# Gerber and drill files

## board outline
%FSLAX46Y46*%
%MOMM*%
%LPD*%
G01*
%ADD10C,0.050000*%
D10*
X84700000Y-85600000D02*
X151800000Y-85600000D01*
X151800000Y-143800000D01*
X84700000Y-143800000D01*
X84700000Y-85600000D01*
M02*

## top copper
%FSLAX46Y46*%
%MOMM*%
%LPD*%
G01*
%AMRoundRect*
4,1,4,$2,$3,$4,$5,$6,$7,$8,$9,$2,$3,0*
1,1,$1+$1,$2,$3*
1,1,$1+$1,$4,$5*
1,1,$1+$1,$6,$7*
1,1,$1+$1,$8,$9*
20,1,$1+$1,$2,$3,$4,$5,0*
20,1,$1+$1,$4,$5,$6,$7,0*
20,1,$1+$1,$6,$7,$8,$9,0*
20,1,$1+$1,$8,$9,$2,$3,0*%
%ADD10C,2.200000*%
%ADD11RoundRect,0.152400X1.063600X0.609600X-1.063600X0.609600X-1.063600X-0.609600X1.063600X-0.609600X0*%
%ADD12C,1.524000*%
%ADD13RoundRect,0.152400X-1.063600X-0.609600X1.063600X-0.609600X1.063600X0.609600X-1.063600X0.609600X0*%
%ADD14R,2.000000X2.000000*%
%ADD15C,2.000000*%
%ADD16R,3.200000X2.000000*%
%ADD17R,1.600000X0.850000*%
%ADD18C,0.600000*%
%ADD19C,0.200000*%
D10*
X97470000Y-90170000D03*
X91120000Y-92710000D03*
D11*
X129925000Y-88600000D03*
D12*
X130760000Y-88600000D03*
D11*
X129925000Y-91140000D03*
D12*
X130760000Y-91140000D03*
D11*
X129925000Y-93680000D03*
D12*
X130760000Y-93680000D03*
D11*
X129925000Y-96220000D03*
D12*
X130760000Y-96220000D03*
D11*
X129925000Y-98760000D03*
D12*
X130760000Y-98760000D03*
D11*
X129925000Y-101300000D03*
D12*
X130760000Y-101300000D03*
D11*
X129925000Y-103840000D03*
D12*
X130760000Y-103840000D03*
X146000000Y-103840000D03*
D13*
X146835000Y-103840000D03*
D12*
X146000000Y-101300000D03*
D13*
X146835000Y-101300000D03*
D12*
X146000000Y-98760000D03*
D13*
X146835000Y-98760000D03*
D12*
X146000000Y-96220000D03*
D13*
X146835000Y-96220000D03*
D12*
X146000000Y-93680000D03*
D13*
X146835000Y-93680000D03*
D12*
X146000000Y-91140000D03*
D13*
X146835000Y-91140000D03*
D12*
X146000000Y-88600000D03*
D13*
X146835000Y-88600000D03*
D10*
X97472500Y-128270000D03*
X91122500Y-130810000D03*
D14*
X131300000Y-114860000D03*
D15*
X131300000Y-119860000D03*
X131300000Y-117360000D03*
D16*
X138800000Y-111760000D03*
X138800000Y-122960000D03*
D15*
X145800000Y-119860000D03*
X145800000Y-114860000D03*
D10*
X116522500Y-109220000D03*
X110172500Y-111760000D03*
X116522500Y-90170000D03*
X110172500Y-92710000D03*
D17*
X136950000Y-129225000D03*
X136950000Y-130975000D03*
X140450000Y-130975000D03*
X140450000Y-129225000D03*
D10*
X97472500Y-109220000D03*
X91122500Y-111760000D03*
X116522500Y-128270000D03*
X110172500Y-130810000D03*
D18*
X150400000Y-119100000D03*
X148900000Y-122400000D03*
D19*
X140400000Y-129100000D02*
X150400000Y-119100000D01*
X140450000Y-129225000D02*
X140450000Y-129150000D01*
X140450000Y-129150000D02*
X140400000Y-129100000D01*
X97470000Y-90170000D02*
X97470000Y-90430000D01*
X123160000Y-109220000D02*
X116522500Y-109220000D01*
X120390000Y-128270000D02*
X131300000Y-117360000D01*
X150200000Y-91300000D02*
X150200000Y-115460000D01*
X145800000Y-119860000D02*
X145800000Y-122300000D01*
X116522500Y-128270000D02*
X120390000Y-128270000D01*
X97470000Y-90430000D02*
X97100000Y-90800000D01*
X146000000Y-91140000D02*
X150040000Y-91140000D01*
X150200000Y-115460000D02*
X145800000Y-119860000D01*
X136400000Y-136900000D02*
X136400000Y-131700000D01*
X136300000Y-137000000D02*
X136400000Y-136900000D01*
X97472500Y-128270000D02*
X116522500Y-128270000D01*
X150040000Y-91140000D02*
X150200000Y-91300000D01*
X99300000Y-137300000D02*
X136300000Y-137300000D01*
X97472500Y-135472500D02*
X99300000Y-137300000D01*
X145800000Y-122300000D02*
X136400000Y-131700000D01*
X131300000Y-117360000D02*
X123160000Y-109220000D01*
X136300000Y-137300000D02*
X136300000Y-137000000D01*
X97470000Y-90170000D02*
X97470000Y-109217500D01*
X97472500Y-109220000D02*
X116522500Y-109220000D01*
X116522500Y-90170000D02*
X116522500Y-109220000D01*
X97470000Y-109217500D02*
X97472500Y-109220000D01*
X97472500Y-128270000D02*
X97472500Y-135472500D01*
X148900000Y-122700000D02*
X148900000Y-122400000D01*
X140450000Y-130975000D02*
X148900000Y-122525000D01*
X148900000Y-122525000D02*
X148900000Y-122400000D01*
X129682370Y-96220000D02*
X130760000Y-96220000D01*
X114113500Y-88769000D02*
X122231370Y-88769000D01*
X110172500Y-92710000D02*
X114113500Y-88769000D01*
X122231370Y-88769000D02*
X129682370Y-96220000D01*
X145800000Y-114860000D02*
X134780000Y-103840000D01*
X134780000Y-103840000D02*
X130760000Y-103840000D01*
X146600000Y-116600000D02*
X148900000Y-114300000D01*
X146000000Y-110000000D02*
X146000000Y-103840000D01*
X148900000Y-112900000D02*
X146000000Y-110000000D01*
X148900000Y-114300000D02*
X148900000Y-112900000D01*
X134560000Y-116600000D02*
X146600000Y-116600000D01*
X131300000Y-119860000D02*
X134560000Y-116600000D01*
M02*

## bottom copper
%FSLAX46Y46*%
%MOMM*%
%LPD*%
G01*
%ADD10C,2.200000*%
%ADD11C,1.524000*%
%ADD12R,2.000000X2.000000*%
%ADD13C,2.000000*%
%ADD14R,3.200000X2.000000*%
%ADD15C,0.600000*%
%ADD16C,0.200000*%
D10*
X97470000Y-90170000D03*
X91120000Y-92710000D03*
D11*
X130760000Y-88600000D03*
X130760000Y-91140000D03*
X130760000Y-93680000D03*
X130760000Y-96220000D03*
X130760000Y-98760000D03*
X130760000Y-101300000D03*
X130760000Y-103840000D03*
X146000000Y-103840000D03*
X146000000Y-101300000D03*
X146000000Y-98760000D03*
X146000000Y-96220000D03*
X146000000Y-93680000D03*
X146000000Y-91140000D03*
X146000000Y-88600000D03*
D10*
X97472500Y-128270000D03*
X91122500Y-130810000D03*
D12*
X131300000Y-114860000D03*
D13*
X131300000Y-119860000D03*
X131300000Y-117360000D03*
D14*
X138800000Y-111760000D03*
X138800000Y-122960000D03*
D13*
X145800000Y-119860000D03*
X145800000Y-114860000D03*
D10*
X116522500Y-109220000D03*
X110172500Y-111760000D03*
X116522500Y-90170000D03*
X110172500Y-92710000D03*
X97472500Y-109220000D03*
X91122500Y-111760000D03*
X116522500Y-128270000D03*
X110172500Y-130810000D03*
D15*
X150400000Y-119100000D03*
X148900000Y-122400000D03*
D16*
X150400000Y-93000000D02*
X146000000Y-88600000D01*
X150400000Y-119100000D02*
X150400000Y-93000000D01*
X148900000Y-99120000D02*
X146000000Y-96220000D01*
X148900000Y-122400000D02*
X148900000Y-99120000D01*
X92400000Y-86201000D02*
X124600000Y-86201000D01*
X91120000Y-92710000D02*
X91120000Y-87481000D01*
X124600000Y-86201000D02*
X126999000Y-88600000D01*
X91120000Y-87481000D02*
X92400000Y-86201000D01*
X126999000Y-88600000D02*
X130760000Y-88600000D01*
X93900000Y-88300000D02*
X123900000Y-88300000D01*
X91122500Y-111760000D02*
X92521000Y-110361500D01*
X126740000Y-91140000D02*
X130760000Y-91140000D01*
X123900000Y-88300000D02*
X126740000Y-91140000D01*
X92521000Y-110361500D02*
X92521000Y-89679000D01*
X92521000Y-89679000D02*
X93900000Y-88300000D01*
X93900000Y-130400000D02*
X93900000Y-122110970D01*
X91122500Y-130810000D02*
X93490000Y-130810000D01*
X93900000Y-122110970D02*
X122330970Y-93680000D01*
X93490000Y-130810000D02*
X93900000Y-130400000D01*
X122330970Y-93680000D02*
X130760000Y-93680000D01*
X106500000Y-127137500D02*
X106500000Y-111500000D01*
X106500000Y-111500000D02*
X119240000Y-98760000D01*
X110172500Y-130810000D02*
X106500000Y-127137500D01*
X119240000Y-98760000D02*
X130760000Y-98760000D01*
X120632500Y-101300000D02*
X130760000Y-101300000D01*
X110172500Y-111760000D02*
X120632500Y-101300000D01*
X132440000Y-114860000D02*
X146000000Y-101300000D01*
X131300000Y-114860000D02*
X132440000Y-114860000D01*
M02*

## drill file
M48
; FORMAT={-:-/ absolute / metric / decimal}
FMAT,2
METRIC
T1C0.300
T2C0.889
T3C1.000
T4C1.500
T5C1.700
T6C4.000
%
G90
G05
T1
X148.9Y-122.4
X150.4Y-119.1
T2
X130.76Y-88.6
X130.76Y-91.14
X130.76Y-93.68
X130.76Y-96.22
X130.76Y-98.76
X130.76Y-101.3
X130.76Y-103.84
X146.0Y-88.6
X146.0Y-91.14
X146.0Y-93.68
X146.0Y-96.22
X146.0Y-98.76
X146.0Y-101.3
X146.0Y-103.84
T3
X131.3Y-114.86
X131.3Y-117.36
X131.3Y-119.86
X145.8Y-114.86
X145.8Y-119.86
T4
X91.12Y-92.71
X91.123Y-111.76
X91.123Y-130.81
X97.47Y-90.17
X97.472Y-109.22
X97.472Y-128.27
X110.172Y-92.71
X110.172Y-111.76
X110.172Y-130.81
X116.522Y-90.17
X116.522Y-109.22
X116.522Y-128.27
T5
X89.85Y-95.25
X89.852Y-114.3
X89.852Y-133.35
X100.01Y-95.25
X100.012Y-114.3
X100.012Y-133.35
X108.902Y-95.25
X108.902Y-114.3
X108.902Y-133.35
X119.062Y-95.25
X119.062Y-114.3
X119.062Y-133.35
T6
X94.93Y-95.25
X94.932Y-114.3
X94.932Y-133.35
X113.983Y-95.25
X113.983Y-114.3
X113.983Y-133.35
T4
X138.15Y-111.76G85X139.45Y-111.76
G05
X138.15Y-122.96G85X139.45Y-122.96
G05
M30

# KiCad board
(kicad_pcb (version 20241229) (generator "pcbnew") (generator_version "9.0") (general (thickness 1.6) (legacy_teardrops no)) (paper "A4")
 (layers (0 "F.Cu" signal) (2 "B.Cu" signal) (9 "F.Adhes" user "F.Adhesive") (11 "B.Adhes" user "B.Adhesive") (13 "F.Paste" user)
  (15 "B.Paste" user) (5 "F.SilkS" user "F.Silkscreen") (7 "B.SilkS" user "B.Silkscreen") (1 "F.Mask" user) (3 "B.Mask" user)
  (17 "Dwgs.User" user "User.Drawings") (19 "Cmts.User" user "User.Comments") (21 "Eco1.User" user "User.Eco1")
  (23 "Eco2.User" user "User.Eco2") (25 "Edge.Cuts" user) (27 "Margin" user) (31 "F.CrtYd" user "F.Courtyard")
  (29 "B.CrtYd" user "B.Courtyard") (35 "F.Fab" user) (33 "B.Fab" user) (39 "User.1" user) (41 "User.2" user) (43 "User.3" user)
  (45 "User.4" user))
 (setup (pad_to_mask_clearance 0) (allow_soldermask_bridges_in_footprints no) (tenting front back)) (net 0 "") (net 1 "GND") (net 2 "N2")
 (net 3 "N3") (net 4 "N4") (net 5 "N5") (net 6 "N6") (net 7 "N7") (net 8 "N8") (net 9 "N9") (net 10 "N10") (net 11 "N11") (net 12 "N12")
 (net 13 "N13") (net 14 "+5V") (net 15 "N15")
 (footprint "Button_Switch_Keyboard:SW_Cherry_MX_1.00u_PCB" (layer "F.Cu") (at 97.47 90.17)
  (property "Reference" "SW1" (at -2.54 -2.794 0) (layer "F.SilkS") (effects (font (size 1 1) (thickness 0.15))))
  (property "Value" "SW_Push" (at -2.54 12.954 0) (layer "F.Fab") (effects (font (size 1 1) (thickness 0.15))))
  (pad "" np_thru_hole circle (at -7.62 5.08) (size 1.7 1.7) (drill 1.7) (layers "*.Cu" "*.Mask"))
  (pad "" np_thru_hole circle (at -2.54 5.08) (size 4 4) (drill 4) (layers "*.Cu" "*.Mask"))
  (pad "" np_thru_hole circle (at 2.54 5.08) (size 1.7 1.7) (drill 1.7) (layers "*.Cu" "*.Mask"))
  (pad "1" thru_hole circle (at 0 0) (size 2.2 2.2) (drill 1.5) (layers "*.Cu" "*.Mask") (remove_unused_layers no) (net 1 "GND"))
  (pad "2" thru_hole circle (at -6.35 2.54) (size 2.2 2.2) (drill 1.5) (layers "*.Cu" "*.Mask") (remove_unused_layers no) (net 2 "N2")))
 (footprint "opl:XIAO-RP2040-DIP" (layer "F.Cu") (at 138.38 96.22)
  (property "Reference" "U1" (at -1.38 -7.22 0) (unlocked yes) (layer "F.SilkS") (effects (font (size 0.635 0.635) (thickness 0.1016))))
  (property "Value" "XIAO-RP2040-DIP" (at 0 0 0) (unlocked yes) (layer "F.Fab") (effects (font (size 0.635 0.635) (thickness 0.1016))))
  (pad "1" smd roundrect (at -8.455 -7.62 180) (size 2.432 1.524) (layers "F.Cu" "F.Mask") (roundrect_rratio 0.1) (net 2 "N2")
   (thermal_bridge_angle 45))
  (pad "1" thru_hole circle (at -7.62 -7.62 180) (size 1.524 1.524) (drill 0.889) (layers "*.Cu" "*.Mask") (remove_unused_layers no)
   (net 2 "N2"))
  (pad "2" smd roundrect (at -8.455 -5.08 180) (size 2.432 1.524) (layers "F.Cu" "F.Mask") (roundrect_rratio 0.1) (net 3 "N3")
   (thermal_bridge_angle 45))
  (pad "2" thru_hole circle (at -7.62 -5.08 180) (size 1.524 1.524) (drill 0.889) (layers "*.Cu" "*.Mask") (remove_unused_layers no)
   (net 3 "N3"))
  (pad "3" smd roundrect (at -8.455 -2.54 180) (size 2.432 1.524) (layers "F.Cu" "F.Mask") (roundrect_rratio 0.1) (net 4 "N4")
   (thermal_bridge_angle 45))
  (pad "3" thru_hole circle (at -7.62 -2.54 180) (size 1.524 1.524) (drill 0.889) (layers "*.Cu" "*.Mask") (remove_unused_layers no)
   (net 4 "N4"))
  (pad "4" smd roundrect (at -8.455 0 180) (size 2.432 1.524) (layers "F.Cu" "F.Mask") (roundrect_rratio 0.1) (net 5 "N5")
   (thermal_bridge_angle 45))
  (pad "4" thru_hole circle (at -7.62 0 180) (size 1.524 1.524) (drill 0.889) (layers "*.Cu" "*.Mask") (remove_unused_layers no)
   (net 5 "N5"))
  (pad "5" smd roundrect (at -8.455 2.54 180) (size 2.432 1.524) (layers "F.Cu" "F.Mask") (roundrect_rratio 0.1) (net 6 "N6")
   (thermal_bridge_angle 45))
  (pad "5" thru_hole circle (at -7.62 2.54 180) (size 1.524 1.524) (drill 0.889) (layers "*.Cu" "*.Mask") (remove_unused_layers no)
   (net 6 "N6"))
  (pad "6" smd roundrect (at -8.455 5.08 180) (size 2.432 1.524) (layers "F.Cu" "F.Mask") (roundrect_rratio 0.1) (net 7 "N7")
   (thermal_bridge_angle 45))
  (pad "6" thru_hole circle (at -7.62 5.08 180) (size 1.524 1.524) (drill 0.889) (layers "*.Cu" "*.Mask") (remove_unused_layers no)
   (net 7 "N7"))
  (pad "7" smd roundrect (at -8.455 7.62 180) (size 2.432 1.524) (layers "F.Cu" "F.Mask") (roundrect_rratio 0.1) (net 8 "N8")
   (thermal_bridge_angle 45))
  (pad "7" thru_hole circle (at -7.62 7.62 180) (size 1.524 1.524) (drill 0.889) (layers "*.Cu" "*.Mask") (remove_unused_layers no)
   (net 8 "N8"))
  (pad "8" thru_hole circle (at 7.62 7.62) (size 1.524 1.524) (drill 0.889) (layers "*.Cu" "*.Mask") (remove_unused_layers no) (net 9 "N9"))
  (pad "8" smd roundrect (at 8.455 7.62) (size 2.432 1.524) (layers "F.Cu" "F.Mask") (roundrect_rratio 0.1) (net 9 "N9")
   (thermal_bridge_angle 45))
  (pad "9" thru_hole circle (at 7.62 5.08) (size 1.524 1.524) (drill 0.889) (layers "*.Cu" "*.Mask") (remove_unused_layers no)
   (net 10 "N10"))
  (pad "9" smd roundrect (at 8.455 5.08) (size 2.432 1.524) (layers "F.Cu" "F.Mask") (roundrect_rratio 0.1) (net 10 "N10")
   (thermal_bridge_angle 45))
  (pad "10" thru_hole circle (at 7.62 2.54) (size 1.524 1.524) (drill 0.889) (layers "*.Cu" "*.Mask") (remove_unused_layers no)
   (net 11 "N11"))
  (pad "10" smd roundrect (at 8.455 2.54) (size 2.432 1.524) (layers "F.Cu" "F.Mask") (roundrect_rratio 0.1) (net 11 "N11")
   (thermal_bridge_angle 45))
  (pad "11" thru_hole circle (at 7.62 0) (size 1.524 1.524) (drill 0.889) (layers "*.Cu" "*.Mask") (remove_unused_layers no) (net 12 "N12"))
  (pad "11" smd roundrect (at 8.455 0) (size 2.432 1.524) (layers "F.Cu" "F.Mask") (roundrect_rratio 0.1) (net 12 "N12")
   (thermal_bridge_angle 45))
  (pad "12" thru_hole circle (at 7.62 -2.54) (size 1.524 1.524) (drill 0.889) (layers "*.Cu" "*.Mask") (remove_unused_layers no)
   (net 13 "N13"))
  (pad "12" smd roundrect (at 8.455 -2.54) (size 2.432 1.524) (layers "F.Cu" "F.Mask") (roundrect_rratio 0.1) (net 13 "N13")
   (thermal_bridge_angle 45))
  (pad "13" thru_hole circle (at 7.62 -5.08) (size 1.524 1.524) (drill 0.889) (layers "*.Cu" "*.Mask") (remove_unused_layers no)
   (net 1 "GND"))
  (pad "13" smd roundrect (at 8.455 -5.08) (size 2.432 1.524) (layers "F.Cu" "F.Mask") (roundrect_rratio 0.1) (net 1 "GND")
   (thermal_bridge_angle 45))
  (pad "14" thru_hole circle (at 7.62 -7.62) (size 1.524 1.524) (drill 0.889) (layers "*.Cu" "*.Mask") (remove_unused_layers no)
   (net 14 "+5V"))
  (pad "14" smd roundrect (at 8.455 -7.62) (size 2.432 1.524) (layers "F.Cu" "F.Mask") (roundrect_rratio 0.1) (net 14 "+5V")
   (thermal_bridge_angle 45)))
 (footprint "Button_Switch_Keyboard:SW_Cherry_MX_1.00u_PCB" (layer "F.Cu") (at 97.4725 128.27)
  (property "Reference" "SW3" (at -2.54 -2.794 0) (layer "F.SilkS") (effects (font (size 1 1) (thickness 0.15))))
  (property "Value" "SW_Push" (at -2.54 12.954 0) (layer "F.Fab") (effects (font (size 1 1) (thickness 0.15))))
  (pad "" np_thru_hole circle (at -7.62 5.08) (size 1.7 1.7) (drill 1.7) (layers "*.Cu" "*.Mask"))
  (pad "" np_thru_hole circle (at -2.54 5.08) (size 4 4) (drill 4) (layers "*.Cu" "*.Mask"))
  (pad "" np_thru_hole circle (at 2.54 5.08) (size 1.7 1.7) (drill 1.7) (layers "*.Cu" "*.Mask"))
  (pad "1" thru_hole circle (at 0 0) (size 2.2 2.2) (drill 1.5) (layers "*.Cu" "*.Mask") (remove_unused_layers no) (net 1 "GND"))
  (pad "2" thru_hole circle (at -6.35 2.54) (size 2.2 2.2) (drill 1.5) (layers "*.Cu" "*.Mask") (remove_unused_layers no) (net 4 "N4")))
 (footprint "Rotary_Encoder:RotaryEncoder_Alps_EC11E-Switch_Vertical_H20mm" (layer "F.Cu") (at 131.3 114.86)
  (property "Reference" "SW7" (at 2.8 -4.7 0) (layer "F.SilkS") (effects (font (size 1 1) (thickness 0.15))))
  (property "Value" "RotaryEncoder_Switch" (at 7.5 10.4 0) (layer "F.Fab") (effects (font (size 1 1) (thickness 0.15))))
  (pad "A" thru_hole rect (at 0 0) (size 2 2) (drill 1) (layers "*.Cu" "*.Mask") (remove_unused_layers no) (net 10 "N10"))
  (pad "B" thru_hole circle (at 0 5) (size 2 2) (drill 1) (layers "*.Cu" "*.Mask") (remove_unused_layers no) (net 9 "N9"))
  (pad "C" thru_hole circle (at 0 2.5) (size 2 2) (drill 1) (layers "*.Cu" "*.Mask") (remove_unused_layers no) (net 1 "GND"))
  (pad "MP" thru_hole rect (at 7.5 -3.1) (size 3.2 2) (drill oval 2.8 1.5) (layers "*.Cu" "*.Mask") (remove_unused_layers no))
  (pad "MP" thru_hole rect (at 7.5 8.1) (size 3.2 2) (drill oval 2.8 1.5) (layers "*.Cu" "*.Mask") (remove_unused_layers no))
  (pad "S1" thru_hole circle (at 14.5 5) (size 2 2) (drill 1) (layers "*.Cu" "*.Mask") (remove_unused_layers no) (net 1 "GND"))
  (pad "S2" thru_hole circle (at 14.5 0) (size 2 2) (drill 1) (layers "*.Cu" "*.Mask") (remove_unused_layers no) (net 8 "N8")))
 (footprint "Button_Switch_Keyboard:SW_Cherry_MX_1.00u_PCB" (layer "F.Cu") (at 116.5225 109.22)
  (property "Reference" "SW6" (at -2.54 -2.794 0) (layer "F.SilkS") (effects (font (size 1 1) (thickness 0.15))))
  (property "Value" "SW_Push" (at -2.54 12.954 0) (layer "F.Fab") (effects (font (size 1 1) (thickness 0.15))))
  (pad "" np_thru_hole circle (at -7.62 5.08) (size 1.7 1.7) (drill 1.7) (layers "*.Cu" "*.Mask"))
  (pad "" np_thru_hole circle (at -2.54 5.08) (size 4 4) (drill 4) (layers "*.Cu" "*.Mask"))
  (pad "" np_thru_hole circle (at 2.54 5.08) (size 1.7 1.7) (drill 1.7) (layers "*.Cu" "*.Mask"))
  (pad "1" thru_hole circle (at 0 0) (size 2.2 2.2) (drill 1.5) (layers "*.Cu" "*.Mask") (remove_unused_layers no) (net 1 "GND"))
  (pad "2" thru_hole circle (at -6.35 2.54) (size 2.2 2.2) (drill 1.5) (layers "*.Cu" "*.Mask") (remove_unused_layers no) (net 7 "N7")))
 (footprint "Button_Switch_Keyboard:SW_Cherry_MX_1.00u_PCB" (layer "F.Cu") (at 116.5225 90.17)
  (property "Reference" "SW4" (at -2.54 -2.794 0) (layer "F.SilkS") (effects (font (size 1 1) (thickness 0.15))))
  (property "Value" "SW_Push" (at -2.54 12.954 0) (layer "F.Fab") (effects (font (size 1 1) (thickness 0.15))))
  (pad "" np_thru_hole circle (at -7.62 5.08) (size 1.7 1.7) (drill 1.7) (layers "*.Cu" "*.Mask"))
  (pad "" np_thru_hole circle (at -2.54 5.08) (size 4 4) (drill 4) (layers "*.Cu" "*.Mask"))
  (pad "" np_thru_hole circle (at 2.54 5.08) (size 1.7 1.7) (drill 1.7) (layers "*.Cu" "*.Mask"))
  (pad "1" thru_hole circle (at 0 0) (size 2.2 2.2) (drill 1.5) (layers "*.Cu" "*.Mask") (remove_unused_layers no) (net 1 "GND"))
  (pad "2" thru_hole circle (at -6.35 2.54) (size 2.2 2.2) (drill 1.5) (layers "*.Cu" "*.Mask") (remove_unused_layers no) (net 5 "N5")))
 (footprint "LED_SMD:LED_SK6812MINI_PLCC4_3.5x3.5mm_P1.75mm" (layer "F.Cu") (at 138.7 130.1)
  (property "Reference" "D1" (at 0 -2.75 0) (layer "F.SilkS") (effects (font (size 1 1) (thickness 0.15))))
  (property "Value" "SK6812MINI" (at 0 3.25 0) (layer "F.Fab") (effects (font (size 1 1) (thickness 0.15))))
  (pad "1" smd rect (at -1.75 -0.875) (size 1.6 0.85) (layers "F.Cu" "F.Mask" "F.Paste") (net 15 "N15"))
  (pad "2" smd rect (at -1.75 0.875) (size 1.6 0.85) (layers "F.Cu" "F.Mask" "F.Paste") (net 1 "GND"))
  (pad "3" smd rect (at 1.75 0.875) (size 1.6 0.85) (layers "F.Cu" "F.Mask" "F.Paste") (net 12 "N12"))
  (pad "4" smd rect (at 1.75 -0.875) (size 1.6 0.85) (layers "F.Cu" "F.Mask" "F.Paste") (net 14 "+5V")))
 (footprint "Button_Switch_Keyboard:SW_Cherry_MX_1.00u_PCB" (layer "F.Cu") (at 97.4725 109.22)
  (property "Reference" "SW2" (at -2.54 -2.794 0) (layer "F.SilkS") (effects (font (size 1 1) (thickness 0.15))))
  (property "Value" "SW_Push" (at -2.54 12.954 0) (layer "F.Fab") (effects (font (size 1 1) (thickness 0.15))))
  (pad "" np_thru_hole circle (at -7.62 5.08) (size 1.7 1.7) (drill 1.7) (layers "*.Cu" "*.Mask"))
  (pad "" np_thru_hole circle (at -2.54 5.08) (size 4 4) (drill 4) (layers "*.Cu" "*.Mask"))
  (pad "" np_thru_hole circle (at 2.54 5.08) (size 1.7 1.7) (drill 1.7) (layers "*.Cu" "*.Mask"))
  (pad "1" thru_hole circle (at 0 0) (size 2.2 2.2) (drill 1.5) (layers "*.Cu" "*.Mask") (remove_unused_layers no) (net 1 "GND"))
  (pad "2" thru_hole circle (at -6.35 2.54) (size 2.2 2.2) (drill 1.5) (layers "*.Cu" "*.Mask") (remove_unused_layers no) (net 3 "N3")))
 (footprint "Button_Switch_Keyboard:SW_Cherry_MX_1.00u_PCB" (layer "F.Cu") (at 116.5225 128.27)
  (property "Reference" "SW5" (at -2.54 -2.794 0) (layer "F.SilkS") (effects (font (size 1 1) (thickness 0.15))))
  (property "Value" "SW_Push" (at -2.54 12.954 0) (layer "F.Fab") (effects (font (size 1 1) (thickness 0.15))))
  (pad "" np_thru_hole circle (at -7.62 5.08) (size 1.7 1.7) (drill 1.7) (layers "*.Cu" "*.Mask"))
  (pad "" np_thru_hole circle (at -2.54 5.08) (size 4 4) (drill 4) (layers "*.Cu" "*.Mask"))
  (pad "" np_thru_hole circle (at 2.54 5.08) (size 1.7 1.7) (drill 1.7) (layers "*.Cu" "*.Mask"))
  (pad "1" thru_hole circle (at 0 0) (size 2.2 2.2) (drill 1.5) (layers "*.Cu" "*.Mask") (remove_unused_layers no) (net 1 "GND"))
  (pad "2" thru_hole circle (at -6.35 2.54) (size 2.2 2.2) (drill 1.5) (layers "*.Cu" "*.Mask") (remove_unused_layers no) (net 6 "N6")))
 (gr_rect (start 84.7 85.6) (end 151.8 143.8) (stroke (width 0.05) (type default)) (fill no) (layer "Edge.Cuts"))
 (segment (start 140.4 129.1) (end 150.4 119.1) (width 0.2) (layer "F.Cu") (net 14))
 (segment (start 140.45 129.225) (end 140.45 129.15) (width 0.2) (layer "F.Cu") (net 14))
 (segment (start 140.45 129.15) (end 140.4 129.1) (width 0.2) (layer "F.Cu") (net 14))
 (via (at 150.4 119.1) (size 0.6) (drill 0.3) (layers "F.Cu" "B.Cu") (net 14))
 (segment (start 150.4 93) (end 146 88.6) (width 0.2) (layer "B.Cu") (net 14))
 (segment (start 150.4 119.1) (end 150.4 93) (width 0.2) (layer "B.Cu") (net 14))
 (segment (start 97.47 90.17) (end 97.47 90.43) (width 0.2) (layer "F.Cu") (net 1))
 (segment (start 123.16 109.22) (end 116.5225 109.22) (width 0.2) (layer "F.Cu") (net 1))
 (segment (start 120.39 128.27) (end 131.3 117.36) (width 0.2) (layer "F.Cu") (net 1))
 (segment (start 150.2 91.3) (end 150.2 115.46) (width 0.2) (layer "F.Cu") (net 1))
 (segment (start 145.8 119.86) (end 145.8 122.3) (width 0.2) (layer "F.Cu") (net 1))
 (segment (start 116.5225 128.27) (end 120.39 128.27) (width 0.2) (layer "F.Cu") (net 1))
 (segment (start 97.47 90.43) (end 97.1 90.8) (width 0.2) (layer "F.Cu") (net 1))
 (segment (start 146 91.14) (end 150.04 91.14) (width 0.2) (layer "F.Cu") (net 1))
 (segment (start 150.2 115.46) (end 145.8 119.86) (width 0.2) (layer "F.Cu") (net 1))
 (segment (start 136.4 136.9) (end 136.4 131.7) (width 0.2) (layer "F.Cu") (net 1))
 (segment (start 136.3 137) (end 136.4 136.9) (width 0.2) (layer "F.Cu") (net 1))
 (segment (start 97.4725 128.27) (end 116.5225 128.27) (width 0.2) (layer "F.Cu") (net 1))
 (segment (start 150.04 91.14) (end 150.2 91.3) (width 0.2) (layer "F.Cu") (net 1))
 (segment (start 99.3 137.3) (end 136.3 137.3) (width 0.2) (layer "F.Cu") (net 1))
 (segment (start 97.4725 135.4725) (end 99.3 137.3) (width 0.2) (layer "F.Cu") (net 1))
 (segment (start 145.8 122.3) (end 136.4 131.7) (width 0.2) (layer "F.Cu") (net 1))
 (segment (start 131.3 117.36) (end 123.16 109.22) (width 0.2) (layer "F.Cu") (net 1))
 (segment (start 136.3 137.3) (end 136.3 137) (width 0.2) (layer "F.Cu") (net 1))
 (segment (start 97.47 90.17) (end 97.47 109.2175) (width 0.2) (layer "F.Cu") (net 1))
 (segment (start 97.4725 109.22) (end 116.5225 109.22) (width 0.2) (layer "F.Cu") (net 1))
 (segment (start 116.5225 90.17) (end 116.5225 109.22) (width 0.2) (layer "F.Cu") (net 1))
 (segment (start 97.47 109.2175) (end 97.4725 109.22) (width 0.2) (layer "F.Cu") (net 1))
 (segment (start 97.4725 128.27) (end 97.4725 135.4725) (width 0.2) (layer "F.Cu") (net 1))
 (segment (start 148.9 122.7) (end 148.9 122.4) (width 0.2) (layer "F.Cu") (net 12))
 (segment (start 140.45 130.975) (end 148.9 122.525) (width 0.2) (layer "F.Cu") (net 12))
 (segment (start 148.9 122.525) (end 148.9 122.4) (width 0.2) (layer "F.Cu") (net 12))
 (via (at 148.9 122.4) (size 0.6) (drill 0.3) (layers "F.Cu" "B.Cu") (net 12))
 (segment (start 148.9 99.12) (end 146 96.22) (width 0.2) (layer "B.Cu") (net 12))
 (segment (start 148.9 122.4) (end 148.9 99.12) (width 0.2) (layer "B.Cu") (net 12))
 (segment (start 92.4 86.201) (end 124.6 86.201) (width 0.2) (layer "B.Cu") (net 2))
 (segment (start 91.12 92.71) (end 91.12 87.481) (width 0.2) (layer "B.Cu") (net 2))
 (segment (start 124.6 86.201) (end 126.999 88.6) (width 0.2) (layer "B.Cu") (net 2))
 (segment (start 91.12 87.481) (end 92.4 86.201) (width 0.2) (layer "B.Cu") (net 2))
 (segment (start 126.999 88.6) (end 130.76 88.6) (width 0.2) (layer "B.Cu") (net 2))
 (segment (start 93.9 88.3) (end 123.9 88.3) (width 0.2) (layer "B.Cu") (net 3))
 (segment (start 91.1225 111.76) (end 92.521 110.3615) (width 0.2) (layer "B.Cu") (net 3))
 (segment (start 126.74 91.14) (end 130.76 91.14) (width 0.2) (layer "B.Cu") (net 3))
 (segment (start 123.9 88.3) (end 126.74 91.14) (width 0.2) (layer "B.Cu") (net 3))
 (segment (start 92.521 110.3615) (end 92.521 89.679) (width 0.2) (layer "B.Cu") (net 3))
 (segment (start 92.521 89.679) (end 93.9 88.3) (width 0.2) (layer "B.Cu") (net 3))
 (segment (start 93.9 130.4) (end 93.9 122.11097) (width 0.2) (layer "B.Cu") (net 4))
 (segment (start 91.1225 130.81) (end 93.49 130.81) (width 0.2) (layer "B.Cu") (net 4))
 (segment (start 93.9 122.11097) (end 122.33097 93.68) (width 0.2) (layer "B.Cu") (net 4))
 (segment (start 93.49 130.81) (end 93.9 130.4) (width 0.2) (layer "B.Cu") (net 4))
 (segment (start 122.33097 93.68) (end 130.76 93.68) (width 0.2) (layer "B.Cu") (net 4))
 (segment (start 129.68237 96.22) (end 130.76 96.22) (width 0.2) (layer "F.Cu") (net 5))
 (segment (start 114.1135 88.769) (end 122.23137 88.769) (width 0.2) (layer "F.Cu") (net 5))
 (segment (start 110.1725 92.71) (end 114.1135 88.769) (width 0.2) (layer "F.Cu") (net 5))
 (segment (start 122.23137 88.769) (end 129.68237 96.22) (width 0.2) (layer "F.Cu") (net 5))
 (segment (start 106.5 127.1375) (end 106.5 111.5) (width 0.2) (layer "B.Cu") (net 6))
 (segment (start 106.5 111.5) (end 119.24 98.76) (width 0.2) (layer "B.Cu") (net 6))
 (segment (start 110.1725 130.81) (end 106.5 127.1375) (width 0.2) (layer "B.Cu") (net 6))
 (segment (start 119.24 98.76) (end 130.76 98.76) (width 0.2) (layer "B.Cu") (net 6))
 (segment (start 120.6325 101.3) (end 130.76 101.3) (width 0.2) (layer "B.Cu") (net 7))
 (segment (start 110.1725 111.76) (end 120.6325 101.3) (width 0.2) (layer "B.Cu") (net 7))
 (segment (start 145.8 114.86) (end 134.78 103.84) (width 0.2) (layer "F.Cu") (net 8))
 (segment (start 134.78 103.84) (end 130.76 103.84) (width 0.2) (layer "F.Cu") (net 8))
 (segment (start 146.6 116.6) (end 148.9 114.3) (width 0.2) (layer "F.Cu") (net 9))
 (segment (start 146 110) (end 146 103.84) (width 0.2) (layer "F.Cu") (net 9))
 (segment (start 148.9 112.9) (end 146 110) (width 0.2) (layer "F.Cu") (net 9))
 (segment (start 148.9 114.3) (end 148.9 112.9) (width 0.2) (layer "F.Cu") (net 9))
 (segment (start 134.56 116.6) (end 146.6 116.6) (width 0.2) (layer "F.Cu") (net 9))
 (segment (start 131.3 119.86) (end 134.56 116.6) (width 0.2) (layer "F.Cu") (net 9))
 (segment (start 132.44 114.86) (end 146 101.3) (width 0.2) (layer "B.Cu") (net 10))
 (segment (start 131.3 114.86) (end 132.44 114.86) (width 0.2) (layer "B.Cu") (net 10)))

